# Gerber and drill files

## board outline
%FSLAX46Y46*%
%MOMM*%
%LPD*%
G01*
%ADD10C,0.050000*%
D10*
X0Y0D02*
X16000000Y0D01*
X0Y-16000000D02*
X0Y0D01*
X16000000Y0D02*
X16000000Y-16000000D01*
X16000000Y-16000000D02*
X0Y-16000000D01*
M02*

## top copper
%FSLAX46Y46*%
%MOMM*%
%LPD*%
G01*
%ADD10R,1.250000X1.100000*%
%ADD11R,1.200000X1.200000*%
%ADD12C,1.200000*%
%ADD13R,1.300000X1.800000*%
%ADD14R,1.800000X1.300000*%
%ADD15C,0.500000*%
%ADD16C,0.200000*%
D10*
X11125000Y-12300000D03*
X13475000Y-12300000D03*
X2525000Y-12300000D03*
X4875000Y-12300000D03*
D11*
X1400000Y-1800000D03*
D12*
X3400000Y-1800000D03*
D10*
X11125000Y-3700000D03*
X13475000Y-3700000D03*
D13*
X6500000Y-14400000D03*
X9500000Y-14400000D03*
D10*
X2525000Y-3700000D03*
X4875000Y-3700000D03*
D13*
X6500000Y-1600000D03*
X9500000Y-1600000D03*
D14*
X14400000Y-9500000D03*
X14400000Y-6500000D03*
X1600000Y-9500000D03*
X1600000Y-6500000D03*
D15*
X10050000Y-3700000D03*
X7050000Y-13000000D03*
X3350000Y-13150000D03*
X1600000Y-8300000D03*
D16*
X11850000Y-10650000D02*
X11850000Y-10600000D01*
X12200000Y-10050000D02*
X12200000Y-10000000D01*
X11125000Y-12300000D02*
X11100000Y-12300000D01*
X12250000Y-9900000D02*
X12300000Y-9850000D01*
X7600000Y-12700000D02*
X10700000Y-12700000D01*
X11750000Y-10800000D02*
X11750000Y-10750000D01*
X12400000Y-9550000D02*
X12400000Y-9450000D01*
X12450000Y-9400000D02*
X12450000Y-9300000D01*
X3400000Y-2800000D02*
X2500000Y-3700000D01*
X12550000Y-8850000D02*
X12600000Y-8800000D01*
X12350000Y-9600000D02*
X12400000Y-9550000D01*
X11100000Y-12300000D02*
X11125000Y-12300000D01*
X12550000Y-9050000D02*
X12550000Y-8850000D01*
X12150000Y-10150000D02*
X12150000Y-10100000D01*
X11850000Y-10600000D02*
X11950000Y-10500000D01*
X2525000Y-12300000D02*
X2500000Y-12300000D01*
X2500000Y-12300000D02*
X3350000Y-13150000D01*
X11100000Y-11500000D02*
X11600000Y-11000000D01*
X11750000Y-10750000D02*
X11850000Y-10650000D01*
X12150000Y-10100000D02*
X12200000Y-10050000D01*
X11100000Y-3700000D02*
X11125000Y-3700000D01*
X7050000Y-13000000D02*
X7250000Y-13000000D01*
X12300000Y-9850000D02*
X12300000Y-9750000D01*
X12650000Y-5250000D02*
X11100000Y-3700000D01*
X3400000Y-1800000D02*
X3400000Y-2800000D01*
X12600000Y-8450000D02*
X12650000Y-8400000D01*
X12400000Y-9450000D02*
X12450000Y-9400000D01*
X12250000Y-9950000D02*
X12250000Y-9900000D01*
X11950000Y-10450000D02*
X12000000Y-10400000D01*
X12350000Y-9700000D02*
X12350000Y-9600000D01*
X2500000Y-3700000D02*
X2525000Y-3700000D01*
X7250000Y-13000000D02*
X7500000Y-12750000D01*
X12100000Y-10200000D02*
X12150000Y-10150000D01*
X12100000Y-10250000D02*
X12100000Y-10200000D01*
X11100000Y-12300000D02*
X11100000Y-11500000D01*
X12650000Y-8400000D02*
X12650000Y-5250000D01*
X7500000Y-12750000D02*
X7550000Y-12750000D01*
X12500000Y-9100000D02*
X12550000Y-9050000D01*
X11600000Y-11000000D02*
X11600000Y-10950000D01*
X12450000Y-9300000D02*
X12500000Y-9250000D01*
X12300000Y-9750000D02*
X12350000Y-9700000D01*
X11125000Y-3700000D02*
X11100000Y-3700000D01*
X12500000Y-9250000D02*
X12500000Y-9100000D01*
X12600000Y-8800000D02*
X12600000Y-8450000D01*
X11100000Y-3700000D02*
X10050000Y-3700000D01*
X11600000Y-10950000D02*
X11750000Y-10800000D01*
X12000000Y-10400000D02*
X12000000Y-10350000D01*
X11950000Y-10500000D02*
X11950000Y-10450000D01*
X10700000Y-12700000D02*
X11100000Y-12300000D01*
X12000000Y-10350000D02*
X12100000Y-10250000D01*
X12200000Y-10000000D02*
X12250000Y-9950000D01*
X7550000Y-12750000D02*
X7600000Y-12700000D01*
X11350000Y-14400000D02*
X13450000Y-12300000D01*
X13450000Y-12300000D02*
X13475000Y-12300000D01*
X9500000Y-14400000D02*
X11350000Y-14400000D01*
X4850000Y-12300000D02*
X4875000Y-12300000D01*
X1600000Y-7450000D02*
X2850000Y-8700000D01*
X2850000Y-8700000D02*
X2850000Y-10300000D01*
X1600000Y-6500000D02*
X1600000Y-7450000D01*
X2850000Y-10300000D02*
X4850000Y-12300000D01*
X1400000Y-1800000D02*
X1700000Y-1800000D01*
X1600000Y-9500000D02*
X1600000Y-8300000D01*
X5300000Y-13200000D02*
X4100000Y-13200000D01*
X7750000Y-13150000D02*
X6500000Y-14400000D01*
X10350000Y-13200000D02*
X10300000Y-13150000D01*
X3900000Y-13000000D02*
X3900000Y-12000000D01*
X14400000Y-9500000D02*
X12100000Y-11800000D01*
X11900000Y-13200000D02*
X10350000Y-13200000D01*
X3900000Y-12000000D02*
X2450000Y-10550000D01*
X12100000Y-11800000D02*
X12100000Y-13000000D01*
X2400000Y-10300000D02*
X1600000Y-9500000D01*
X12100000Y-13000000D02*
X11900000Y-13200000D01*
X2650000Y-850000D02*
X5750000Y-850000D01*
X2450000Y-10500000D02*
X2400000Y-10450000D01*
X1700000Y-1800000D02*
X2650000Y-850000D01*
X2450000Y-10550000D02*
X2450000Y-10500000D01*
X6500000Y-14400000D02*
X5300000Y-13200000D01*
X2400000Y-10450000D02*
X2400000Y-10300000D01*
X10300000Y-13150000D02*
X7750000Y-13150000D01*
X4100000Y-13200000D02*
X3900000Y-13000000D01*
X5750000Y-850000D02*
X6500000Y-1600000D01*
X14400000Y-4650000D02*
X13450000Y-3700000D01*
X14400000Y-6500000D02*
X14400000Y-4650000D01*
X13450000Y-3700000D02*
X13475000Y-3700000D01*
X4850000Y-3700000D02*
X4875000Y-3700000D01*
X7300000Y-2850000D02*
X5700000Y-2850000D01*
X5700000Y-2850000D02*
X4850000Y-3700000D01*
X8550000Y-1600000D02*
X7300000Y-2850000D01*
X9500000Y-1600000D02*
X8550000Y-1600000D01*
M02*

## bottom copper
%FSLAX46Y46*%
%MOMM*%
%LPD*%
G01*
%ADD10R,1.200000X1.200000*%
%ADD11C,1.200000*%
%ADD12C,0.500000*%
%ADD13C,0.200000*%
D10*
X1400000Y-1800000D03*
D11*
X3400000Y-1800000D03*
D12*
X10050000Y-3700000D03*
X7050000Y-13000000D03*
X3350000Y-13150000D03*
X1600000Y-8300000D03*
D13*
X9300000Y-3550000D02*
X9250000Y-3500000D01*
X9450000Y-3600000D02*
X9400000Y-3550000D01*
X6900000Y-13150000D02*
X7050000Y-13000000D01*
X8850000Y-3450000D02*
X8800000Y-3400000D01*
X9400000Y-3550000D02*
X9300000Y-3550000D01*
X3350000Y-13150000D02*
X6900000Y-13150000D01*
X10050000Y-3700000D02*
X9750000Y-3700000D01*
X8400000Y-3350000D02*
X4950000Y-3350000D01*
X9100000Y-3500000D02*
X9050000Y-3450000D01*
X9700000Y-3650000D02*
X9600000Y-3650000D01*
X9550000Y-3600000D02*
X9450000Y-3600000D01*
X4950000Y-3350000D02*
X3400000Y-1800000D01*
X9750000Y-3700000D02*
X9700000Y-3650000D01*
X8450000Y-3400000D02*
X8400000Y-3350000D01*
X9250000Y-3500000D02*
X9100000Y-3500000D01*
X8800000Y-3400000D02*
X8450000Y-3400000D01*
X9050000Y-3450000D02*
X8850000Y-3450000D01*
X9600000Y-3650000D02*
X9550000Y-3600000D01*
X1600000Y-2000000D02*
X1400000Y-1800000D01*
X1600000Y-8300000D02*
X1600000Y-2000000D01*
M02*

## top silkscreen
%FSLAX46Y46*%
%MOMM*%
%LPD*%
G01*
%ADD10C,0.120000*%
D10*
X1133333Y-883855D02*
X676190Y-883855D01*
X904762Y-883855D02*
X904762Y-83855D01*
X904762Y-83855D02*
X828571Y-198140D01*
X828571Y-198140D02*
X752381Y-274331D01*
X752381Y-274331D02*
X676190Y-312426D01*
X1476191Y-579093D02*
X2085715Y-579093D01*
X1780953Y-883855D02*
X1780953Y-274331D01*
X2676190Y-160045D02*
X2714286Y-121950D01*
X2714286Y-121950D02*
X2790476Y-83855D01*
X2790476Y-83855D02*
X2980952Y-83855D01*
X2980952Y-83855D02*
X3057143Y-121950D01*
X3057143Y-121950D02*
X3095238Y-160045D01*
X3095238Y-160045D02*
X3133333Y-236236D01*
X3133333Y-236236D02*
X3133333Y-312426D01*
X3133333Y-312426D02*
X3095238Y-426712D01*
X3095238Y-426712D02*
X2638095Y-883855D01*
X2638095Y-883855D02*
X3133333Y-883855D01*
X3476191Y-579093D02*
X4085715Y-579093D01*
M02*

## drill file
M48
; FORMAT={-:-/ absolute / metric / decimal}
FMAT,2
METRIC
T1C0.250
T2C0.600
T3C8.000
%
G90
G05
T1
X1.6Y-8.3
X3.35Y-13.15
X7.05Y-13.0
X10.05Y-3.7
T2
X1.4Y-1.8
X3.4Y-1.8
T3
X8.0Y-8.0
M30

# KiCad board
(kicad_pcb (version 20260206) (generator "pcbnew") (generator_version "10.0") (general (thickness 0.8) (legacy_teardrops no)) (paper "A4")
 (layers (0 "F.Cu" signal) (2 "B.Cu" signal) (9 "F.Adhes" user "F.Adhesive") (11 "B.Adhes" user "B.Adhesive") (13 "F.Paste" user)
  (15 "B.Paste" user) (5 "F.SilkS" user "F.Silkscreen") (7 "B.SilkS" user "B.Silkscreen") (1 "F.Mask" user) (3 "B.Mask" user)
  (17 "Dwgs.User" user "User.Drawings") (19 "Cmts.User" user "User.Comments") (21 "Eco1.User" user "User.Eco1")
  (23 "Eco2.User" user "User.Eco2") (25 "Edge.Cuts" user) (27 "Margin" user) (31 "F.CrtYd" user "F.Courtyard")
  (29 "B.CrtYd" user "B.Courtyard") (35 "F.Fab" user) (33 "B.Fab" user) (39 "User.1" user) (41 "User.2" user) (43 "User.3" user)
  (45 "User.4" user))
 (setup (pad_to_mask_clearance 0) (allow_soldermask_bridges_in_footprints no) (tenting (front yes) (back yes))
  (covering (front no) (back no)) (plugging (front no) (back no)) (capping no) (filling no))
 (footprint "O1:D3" (layer "F.Cu") (at 12.3 12.3)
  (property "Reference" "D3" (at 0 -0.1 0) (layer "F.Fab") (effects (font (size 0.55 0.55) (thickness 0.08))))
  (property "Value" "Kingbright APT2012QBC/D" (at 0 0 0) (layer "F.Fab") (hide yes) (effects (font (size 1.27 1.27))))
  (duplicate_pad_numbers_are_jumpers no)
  (pad "1" smd rect (at -1.175 0) (size 1.25 1.1) (layers "F.Cu" "F.Mask" "F.Paste") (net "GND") (solder_mask_margin 0.025)
   (thermal_bridge_angle 45))
  (pad "2" smd rect (at 1.175 0) (size 1.25 1.1) (layers "F.Cu" "F.Mask" "F.Paste") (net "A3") (solder_mask_margin 0.025)
   (thermal_bridge_angle 45)))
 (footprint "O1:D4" (layer "F.Cu") (at 3.7 12.3)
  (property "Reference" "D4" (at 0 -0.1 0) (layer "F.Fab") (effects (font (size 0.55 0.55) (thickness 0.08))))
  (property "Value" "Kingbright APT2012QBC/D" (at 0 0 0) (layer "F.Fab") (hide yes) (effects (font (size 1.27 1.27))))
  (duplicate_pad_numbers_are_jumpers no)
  (pad "1" smd rect (at -1.175 0) (size 1.25 1.1) (layers "F.Cu" "F.Mask" "F.Paste") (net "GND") (solder_mask_margin 0.025)
   (thermal_bridge_angle 45))
  (pad "2" smd rect (at 1.175 0) (size 1.25 1.1) (layers "F.Cu" "F.Mask" "F.Paste") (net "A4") (solder_mask_margin 0.025)
   (thermal_bridge_angle 45)))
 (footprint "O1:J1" (layer "F.Cu") (at 2.4 1.8)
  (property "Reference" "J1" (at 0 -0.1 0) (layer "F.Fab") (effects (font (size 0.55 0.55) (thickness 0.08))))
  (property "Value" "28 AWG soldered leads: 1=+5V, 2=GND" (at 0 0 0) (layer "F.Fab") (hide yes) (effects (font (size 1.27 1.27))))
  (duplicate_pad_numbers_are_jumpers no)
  (pad "1" thru_hole rect (at -1 0) (size 1.2 1.2) (drill 0.6) (layers "*.Cu" "*.Mask") (remove_unused_layers no) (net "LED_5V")
   (solder_mask_margin 0.025) (thermal_bridge_angle 45))
  (pad "2" thru_hole circle (at 1 0) (size 1.2 1.2) (drill 0.6) (layers "*.Cu" "*.Mask") (remove_unused_layers no) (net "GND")
   (solder_mask_margin 0.025)))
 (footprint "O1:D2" (layer "F.Cu") (at 12.3 3.7)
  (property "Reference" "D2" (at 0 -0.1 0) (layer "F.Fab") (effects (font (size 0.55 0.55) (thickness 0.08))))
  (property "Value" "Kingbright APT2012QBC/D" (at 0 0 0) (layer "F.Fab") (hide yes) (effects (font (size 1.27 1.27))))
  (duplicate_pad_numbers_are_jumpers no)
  (pad "1" smd rect (at -1.175 0) (size 1.25 1.1) (layers "F.Cu" "F.Mask" "F.Paste") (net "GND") (solder_mask_margin 0.025)
   (thermal_bridge_angle 45))
  (pad "2" smd rect (at 1.175 0) (size 1.25 1.1) (layers "F.Cu" "F.Mask" "F.Paste") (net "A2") (solder_mask_margin 0.025)
   (thermal_bridge_angle 45)))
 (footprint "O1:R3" (layer "F.Cu") (at 8 14.4)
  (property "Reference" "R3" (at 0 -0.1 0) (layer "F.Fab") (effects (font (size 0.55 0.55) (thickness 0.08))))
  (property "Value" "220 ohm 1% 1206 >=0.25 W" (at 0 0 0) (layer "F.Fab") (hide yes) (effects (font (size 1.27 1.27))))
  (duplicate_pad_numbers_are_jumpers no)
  (pad "1" smd rect (at -1.5 0) (size 1.3 1.8) (layers "F.Cu" "F.Mask" "F.Paste") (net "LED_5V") (solder_mask_margin 0.025)
   (thermal_bridge_angle 45))
  (pad "2" smd rect (at 1.5 0) (size 1.3 1.8) (layers "F.Cu" "F.Mask" "F.Paste") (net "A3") (solder_mask_margin 0.025)
   (thermal_bridge_angle 45)))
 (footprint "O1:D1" (layer "F.Cu") (at 3.7 3.7)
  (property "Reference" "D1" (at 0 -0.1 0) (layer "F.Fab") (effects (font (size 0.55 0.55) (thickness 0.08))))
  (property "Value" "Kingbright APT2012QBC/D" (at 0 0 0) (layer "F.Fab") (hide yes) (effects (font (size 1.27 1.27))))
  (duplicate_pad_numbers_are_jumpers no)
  (pad "1" smd rect (at -1.175 0) (size 1.25 1.1) (layers "F.Cu" "F.Mask" "F.Paste") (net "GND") (solder_mask_margin 0.025)
   (thermal_bridge_angle 45))
  (pad "2" smd rect (at 1.175 0) (size 1.25 1.1) (layers "F.Cu" "F.Mask" "F.Paste") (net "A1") (solder_mask_margin 0.025)
   (thermal_bridge_angle 45)))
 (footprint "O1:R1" (layer "F.Cu") (at 8 1.6)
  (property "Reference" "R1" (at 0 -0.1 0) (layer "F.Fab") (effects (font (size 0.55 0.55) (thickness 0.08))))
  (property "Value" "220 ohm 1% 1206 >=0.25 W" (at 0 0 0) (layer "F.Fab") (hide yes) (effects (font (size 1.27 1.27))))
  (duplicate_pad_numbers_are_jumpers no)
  (pad "1" smd rect (at -1.5 0) (size 1.3 1.8) (layers "F.Cu" "F.Mask" "F.Paste") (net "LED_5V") (solder_mask_margin 0.025)
   (thermal_bridge_angle 45))
  (pad "2" smd rect (at 1.5 0) (size 1.3 1.8) (layers "F.Cu" "F.Mask" "F.Paste") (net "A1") (solder_mask_margin 0.025)
   (thermal_bridge_angle 45)))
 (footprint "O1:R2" (layer "F.Cu") (at 14.4 8 90)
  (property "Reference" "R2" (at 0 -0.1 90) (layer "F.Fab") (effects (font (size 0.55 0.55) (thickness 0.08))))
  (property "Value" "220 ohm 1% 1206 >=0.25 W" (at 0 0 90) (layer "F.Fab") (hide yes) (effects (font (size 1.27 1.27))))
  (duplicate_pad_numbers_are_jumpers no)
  (pad "1" smd rect (at -1.5 0 90) (size 1.3 1.8) (layers "F.Cu" "F.Mask" "F.Paste") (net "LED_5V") (solder_mask_margin 0.025)
   (thermal_bridge_angle 45))
  (pad "2" smd rect (at 1.5 0 90) (size 1.3 1.8) (layers "F.Cu" "F.Mask" "F.Paste") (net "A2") (solder_mask_margin 0.025)
   (thermal_bridge_angle 45)))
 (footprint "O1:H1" (layer "F.Cu") (at 8 8)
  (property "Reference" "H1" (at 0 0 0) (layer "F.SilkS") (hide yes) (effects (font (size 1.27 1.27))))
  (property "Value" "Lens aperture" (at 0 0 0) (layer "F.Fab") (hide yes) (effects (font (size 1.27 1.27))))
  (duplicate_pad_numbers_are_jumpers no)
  (pad "" np_thru_hole circle (at 0 0) (size 8 8) (drill 8) (layers "*.Cu" "*.Mask")))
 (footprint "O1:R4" (layer "F.Cu") (at 1.6 8 90)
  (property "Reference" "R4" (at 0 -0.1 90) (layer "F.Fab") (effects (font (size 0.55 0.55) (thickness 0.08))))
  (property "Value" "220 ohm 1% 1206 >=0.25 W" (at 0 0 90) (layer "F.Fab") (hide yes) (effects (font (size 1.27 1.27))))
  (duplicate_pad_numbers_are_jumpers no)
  (pad "1" smd rect (at -1.5 0 90) (size 1.3 1.8) (layers "F.Cu" "F.Mask" "F.Paste") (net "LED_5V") (solder_mask_margin 0.025)
   (thermal_bridge_angle 45))
  (pad "2" smd rect (at 1.5 0 90) (size 1.3 1.8) (layers "F.Cu" "F.Mask" "F.Paste") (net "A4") (solder_mask_margin 0.025)
   (thermal_bridge_angle 45)))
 (gr_line (start 0 0) (end 16 0) (stroke (width 0.05) (type default)) (layer "Edge.Cuts"))
 (gr_line (start 0 16) (end 0 0) (stroke (width 0.05) (type default)) (layer "Edge.Cuts"))
 (gr_line (start 16 0) (end 16 16) (stroke (width 0.05) (type default)) (layer "Edge.Cuts"))
 (gr_line (start 16 16) (end 0 16) (stroke (width 0.05) (type default)) (layer "Edge.Cuts"))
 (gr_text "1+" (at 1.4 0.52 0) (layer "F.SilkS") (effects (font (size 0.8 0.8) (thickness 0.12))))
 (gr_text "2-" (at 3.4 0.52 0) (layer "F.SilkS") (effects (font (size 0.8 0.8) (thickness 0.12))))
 (segment (start 4.85 3.7) (end 4.875 3.7) (width 0.2) (layer "F.Cu") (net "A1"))
 (segment (start 7.3 2.85) (end 5.7 2.85) (width 0.2) (layer "F.Cu") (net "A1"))
 (segment (start 5.7 2.85) (end 4.85 3.7) (width 0.2) (layer "F.Cu") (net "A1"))
 (segment (start 8.55 1.6) (end 7.3 2.85) (width 0.2) (layer "F.Cu") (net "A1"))
 (segment (start 9.5 1.6) (end 8.55 1.6) (width 0.2) (layer "F.Cu") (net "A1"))
 (segment (start 14.4 4.65) (end 13.45 3.7) (width 0.2) (layer "F.Cu") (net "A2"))
 (segment (start 14.4 6.5) (end 14.4 4.65) (width 0.2) (layer "F.Cu") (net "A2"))
 (segment (start 13.45 3.7) (end 13.475 3.7) (width 0.2) (layer "F.Cu") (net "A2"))
 (segment (start 11.35 14.4) (end 13.45 12.3) (width 0.2) (layer "F.Cu") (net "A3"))
 (segment (start 13.45 12.3) (end 13.475 12.3) (width 0.2) (layer "F.Cu") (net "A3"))
 (segment (start 9.5 14.4) (end 11.35 14.4) (width 0.2) (layer "F.Cu") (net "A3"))
 (segment (start 4.85 12.3) (end 4.875 12.3) (width 0.2) (layer "F.Cu") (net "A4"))
 (segment (start 1.6 7.45) (end 2.85 8.7) (width 0.2) (layer "F.Cu") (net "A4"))
 (segment (start 2.85 8.7) (end 2.85 10.3) (width 0.2) (layer "F.Cu") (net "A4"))
 (segment (start 1.6 6.5) (end 1.6 7.45) (width 0.2) (layer "F.Cu") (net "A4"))
 (segment (start 2.85 10.3) (end 4.85 12.3) (width 0.2) (layer "F.Cu") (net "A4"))
 (segment (start 11.85 10.65) (end 11.85 10.6) (width 0.2) (layer "F.Cu") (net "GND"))
 (segment (start 12.2 10.05) (end 12.2 10) (width 0.2) (layer "F.Cu") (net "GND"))
 (segment (start 11.125 12.3) (end 11.1 12.3) (width 0.2) (layer "F.Cu") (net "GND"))
 (segment (start 12.25 9.9) (end 12.3 9.85) (width 0.2) (layer "F.Cu") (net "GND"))
 (segment (start 7.6 12.7) (end 10.7 12.7) (width 0.2) (layer "F.Cu") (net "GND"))
 (segment (start 11.75 10.8) (end 11.75 10.75) (width 0.2) (layer "F.Cu") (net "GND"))
 (segment (start 12.4 9.55) (end 12.4 9.45) (width 0.2) (layer "F.Cu") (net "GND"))
 (segment (start 12.45 9.4) (end 12.45 9.3) (width 0.2) (layer "F.Cu") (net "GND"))
 (segment (start 3.4 2.8) (end 2.5 3.7) (width 0.2) (layer "F.Cu") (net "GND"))
 (segment (start 12.55 8.85) (end 12.6 8.8) (width 0.2) (layer "F.Cu") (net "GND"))
 (segment (start 12.35 9.6) (end 12.4 9.55) (width 0.2) (layer "F.Cu") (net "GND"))
 (segment (start 11.1 12.3) (end 11.125 12.3) (width 0.2) (layer "F.Cu") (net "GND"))
 (segment (start 12.55 9.05) (end 12.55 8.85) (width 0.2) (layer "F.Cu") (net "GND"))
 (segment (start 12.15 10.15) (end 12.15 10.1) (width 0.2) (layer "F.Cu") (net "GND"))
 (segment (start 11.85 10.6) (end 11.95 10.5) (width 0.2) (layer "F.Cu") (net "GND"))
 (segment (start 2.525 12.3) (end 2.5 12.3) (width 0.2) (layer "F.Cu") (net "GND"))
 (segment (start 2.5 12.3) (end 3.35 13.15) (width 0.2) (layer "F.Cu") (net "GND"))
 (segment (start 11.1 11.5) (end 11.6 11) (width 0.2) (layer "F.Cu") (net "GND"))
 (segment (start 11.75 10.75) (end 11.85 10.65) (width 0.2) (layer "F.Cu") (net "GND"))
 (segment (start 12.15 10.1) (end 12.2 10.05) (width 0.2) (layer "F.Cu") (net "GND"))
 (segment (start 11.1 3.7) (end 11.125 3.7) (width 0.2) (layer "F.Cu") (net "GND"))
 (segment (start 7.05 13) (end 7.25 13) (width 0.2) (layer "F.Cu") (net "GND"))
 (segment (start 12.3 9.85) (end 12.3 9.75) (width 0.2) (layer "F.Cu") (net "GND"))
 (segment (start 12.65 5.25) (end 11.1 3.7) (width 0.2) (layer "F.Cu") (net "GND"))
 (segment (start 3.4 1.8) (end 3.4 2.8) (width 0.2) (layer "F.Cu") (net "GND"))
 (segment (start 12.6 8.45) (end 12.65 8.4) (width 0.2) (layer "F.Cu") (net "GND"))
 (segment (start 12.4 9.45) (end 12.45 9.4) (width 0.2) (layer "F.Cu") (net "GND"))
 (segment (start 12.25 9.95) (end 12.25 9.9) (width 0.2) (layer "F.Cu") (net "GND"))
 (segment (start 11.95 10.45) (end 12 10.4) (width 0.2) (layer "F.Cu") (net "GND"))
 (segment (start 12.35 9.7) (end 12.35 9.6) (width 0.2) (layer "F.Cu") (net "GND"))
 (segment (start 2.5 3.7) (end 2.525 3.7) (width 0.2) (layer "F.Cu") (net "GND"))
 (segment (start 7.25 13) (end 7.5 12.75) (width 0.2) (layer "F.Cu") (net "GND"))
 (segment (start 12.1 10.2) (end 12.15 10.15) (width 0.2) (layer "F.Cu") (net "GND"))
 (segment (start 12.1 10.25) (end 12.1 10.2) (width 0.2) (layer "F.Cu") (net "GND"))
 (segment (start 11.1 12.3) (end 11.1 11.5) (width 0.2) (layer "F.Cu") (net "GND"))
 (segment (start 12.65 8.4) (end 12.65 5.25) (width 0.2) (layer "F.Cu") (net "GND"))
 (segment (start 7.5 12.75) (end 7.55 12.75) (width 0.2) (layer "F.Cu") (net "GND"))
 (segment (start 12.5 9.1) (end 12.55 9.05) (width 0.2) (layer "F.Cu") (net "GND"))
 (segment (start 11.6 11) (end 11.6 10.95) (width 0.2) (layer "F.Cu") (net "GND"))
 (segment (start 12.45 9.3) (end 12.5 9.25) (width 0.2) (layer "F.Cu") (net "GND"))
 (segment (start 12.3 9.75) (end 12.35 9.7) (width 0.2) (layer "F.Cu") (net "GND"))
 (segment (start 11.125 3.7) (end 11.1 3.7) (width 0.2) (layer "F.Cu") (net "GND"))
 (segment (start 12.5 9.25) (end 12.5 9.1) (width 0.2) (layer "F.Cu") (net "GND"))
 (segment (start 12.6 8.8) (end 12.6 8.45) (width 0.2) (layer "F.Cu") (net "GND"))
 (segment (start 11.1 3.7) (end 10.05 3.7) (width 0.2) (layer "F.Cu") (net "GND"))
 (segment (start 11.6 10.95) (end 11.75 10.8) (width 0.2) (layer "F.Cu") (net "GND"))
 (segment (start 12 10.4) (end 12 10.35) (width 0.2) (layer "F.Cu") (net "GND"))
 (segment (start 11.95 10.5) (end 11.95 10.45) (width 0.2) (layer "F.Cu") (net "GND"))
 (segment (start 10.7 12.7) (end 11.1 12.3) (width 0.2) (layer "F.Cu") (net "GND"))
 (segment (start 12 10.35) (end 12.1 10.25) (width 0.2) (layer "F.Cu") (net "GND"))
 (segment (start 12.2 10) (end 12.25 9.95) (width 0.2) (layer "F.Cu") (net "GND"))
 (segment (start 7.55 12.75) (end 7.6 12.7) (width 0.2) (layer "F.Cu") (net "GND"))
 (via (at 10.05 3.7) (size 0.5) (drill 0.25) (layers "F.Cu" "B.Cu") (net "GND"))
 (via (at 7.05 13) (size 0.5) (drill 0.25) (layers "F.Cu" "B.Cu") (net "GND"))
 (via (at 3.35 13.15) (size 0.5) (drill 0.25) (layers "F.Cu" "B.Cu") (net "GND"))
 (segment (start 9.3 3.55) (end 9.25 3.5) (width 0.2) (layer "B.Cu") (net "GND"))
 (segment (start 9.45 3.6) (end 9.4 3.55) (width 0.2) (layer "B.Cu") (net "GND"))
 (segment (start 6.9 13.15) (end 7.05 13) (width 0.2) (layer "B.Cu") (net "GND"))
 (segment (start 8.85 3.45) (end 8.8 3.4) (width 0.2) (layer "B.Cu") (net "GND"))
 (segment (start 9.4 3.55) (end 9.3 3.55) (width 0.2) (layer "B.Cu") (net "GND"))
 (segment (start 3.35 13.15) (end 6.9 13.15) (width 0.2) (layer "B.Cu") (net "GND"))
 (segment (start 10.05 3.7) (end 9.75 3.7) (width 0.2) (layer "B.Cu") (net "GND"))
 (segment (start 8.4 3.35) (end 4.95 3.35) (width 0.2) (layer "B.Cu") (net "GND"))
 (segment (start 9.1 3.5) (end 9.05 3.45) (width 0.2) (layer "B.Cu") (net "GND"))
 (segment (start 9.7 3.65) (end 9.6 3.65) (width 0.2) (layer "B.Cu") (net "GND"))
 (segment (start 9.55 3.6) (end 9.45 3.6) (width 0.2) (layer "B.Cu") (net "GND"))
 (segment (start 4.95 3.35) (end 3.4 1.8) (width 0.2) (layer "B.Cu") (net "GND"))
 (segment (start 9.75 3.7) (end 9.7 3.65) (width 0.2) (layer "B.Cu") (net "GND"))
 (segment (start 8.45 3.4) (end 8.4 3.35) (width 0.2) (layer "B.Cu") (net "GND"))
 (segment (start 9.25 3.5) (end 9.1 3.5) (width 0.2) (layer "B.Cu") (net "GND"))
 (segment (start 8.8 3.4) (end 8.45 3.4) (width 0.2) (layer "B.Cu") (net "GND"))
 (segment (start 9.05 3.45) (end 8.85 3.45) (width 0.2) (layer "B.Cu") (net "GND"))
 (segment (start 9.6 3.65) (end 9.55 3.6) (width 0.2) (layer "B.Cu") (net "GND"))
 (segment (start 1.4 1.8) (end 1.7 1.8) (width 0.2) (layer "F.Cu") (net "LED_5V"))
 (segment (start 1.6 9.5) (end 1.6 8.3) (width 0.2) (layer "F.Cu") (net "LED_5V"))
 (segment (start 5.3 13.2) (end 4.1 13.2) (width 0.2) (layer "F.Cu") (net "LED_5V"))
 (segment (start 7.75 13.15) (end 6.5 14.4) (width 0.2) (layer "F.Cu") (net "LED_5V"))
 (segment (start 10.35 13.2) (end 10.3 13.15) (width 0.2) (layer "F.Cu") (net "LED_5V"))
 (segment (start 3.9 13) (end 3.9 12) (width 0.2) (layer "F.Cu") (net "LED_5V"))
 (segment (start 14.4 9.5) (end 12.1 11.8) (width 0.2) (layer "F.Cu") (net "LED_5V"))
 (segment (start 11.9 13.2) (end 10.35 13.2) (width 0.2) (layer "F.Cu") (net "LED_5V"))
 (segment (start 3.9 12) (end 2.45 10.55) (width 0.2) (layer "F.Cu") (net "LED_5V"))
 (segment (start 12.1 11.8) (end 12.1 13) (width 0.2) (layer "F.Cu") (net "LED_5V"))
 (segment (start 2.4 10.3) (end 1.6 9.5) (width 0.2) (layer "F.Cu") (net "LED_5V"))
 (segment (start 12.1 13) (end 11.9 13.2) (width 0.2) (layer "F.Cu") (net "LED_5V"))
 (segment (start 2.65 0.85) (end 5.75 0.85) (width 0.2) (layer "F.Cu") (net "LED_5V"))
 (segment (start 2.45 10.5) (end 2.4 10.45) (width 0.2) (layer "F.Cu") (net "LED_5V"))
 (segment (start 1.7 1.8) (end 2.65 0.85) (width 0.2) (layer "F.Cu") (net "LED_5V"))
 (segment (start 2.45 10.55) (end 2.45 10.5) (width 0.2) (layer "F.Cu") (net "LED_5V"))
 (segment (start 6.5 14.4) (end 5.3 13.2) (width 0.2) (layer "F.Cu") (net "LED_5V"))
 (segment (start 2.4 10.45) (end 2.4 10.3) (width 0.2) (layer "F.Cu") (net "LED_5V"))
 (segment (start 10.3 13.15) (end 7.75 13.15) (width 0.2) (layer "F.Cu") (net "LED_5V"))
 (segment (start 4.1 13.2) (end 3.9 13) (width 0.2) (layer "F.Cu") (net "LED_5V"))
 (segment (start 5.75 0.85) (end 6.5 1.6) (width 0.2) (layer "F.Cu") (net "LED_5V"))
 (via (at 1.6 8.3) (size 0.5) (drill 0.25) (layers "F.Cu" "B.Cu") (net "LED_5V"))
 (segment (start 1.6 2) (end 1.4 1.8) (width 0.2) (layer "B.Cu") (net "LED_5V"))
 (segment (start 1.6 8.3) (end 1.6 2) (width 0.2) (layer "B.Cu") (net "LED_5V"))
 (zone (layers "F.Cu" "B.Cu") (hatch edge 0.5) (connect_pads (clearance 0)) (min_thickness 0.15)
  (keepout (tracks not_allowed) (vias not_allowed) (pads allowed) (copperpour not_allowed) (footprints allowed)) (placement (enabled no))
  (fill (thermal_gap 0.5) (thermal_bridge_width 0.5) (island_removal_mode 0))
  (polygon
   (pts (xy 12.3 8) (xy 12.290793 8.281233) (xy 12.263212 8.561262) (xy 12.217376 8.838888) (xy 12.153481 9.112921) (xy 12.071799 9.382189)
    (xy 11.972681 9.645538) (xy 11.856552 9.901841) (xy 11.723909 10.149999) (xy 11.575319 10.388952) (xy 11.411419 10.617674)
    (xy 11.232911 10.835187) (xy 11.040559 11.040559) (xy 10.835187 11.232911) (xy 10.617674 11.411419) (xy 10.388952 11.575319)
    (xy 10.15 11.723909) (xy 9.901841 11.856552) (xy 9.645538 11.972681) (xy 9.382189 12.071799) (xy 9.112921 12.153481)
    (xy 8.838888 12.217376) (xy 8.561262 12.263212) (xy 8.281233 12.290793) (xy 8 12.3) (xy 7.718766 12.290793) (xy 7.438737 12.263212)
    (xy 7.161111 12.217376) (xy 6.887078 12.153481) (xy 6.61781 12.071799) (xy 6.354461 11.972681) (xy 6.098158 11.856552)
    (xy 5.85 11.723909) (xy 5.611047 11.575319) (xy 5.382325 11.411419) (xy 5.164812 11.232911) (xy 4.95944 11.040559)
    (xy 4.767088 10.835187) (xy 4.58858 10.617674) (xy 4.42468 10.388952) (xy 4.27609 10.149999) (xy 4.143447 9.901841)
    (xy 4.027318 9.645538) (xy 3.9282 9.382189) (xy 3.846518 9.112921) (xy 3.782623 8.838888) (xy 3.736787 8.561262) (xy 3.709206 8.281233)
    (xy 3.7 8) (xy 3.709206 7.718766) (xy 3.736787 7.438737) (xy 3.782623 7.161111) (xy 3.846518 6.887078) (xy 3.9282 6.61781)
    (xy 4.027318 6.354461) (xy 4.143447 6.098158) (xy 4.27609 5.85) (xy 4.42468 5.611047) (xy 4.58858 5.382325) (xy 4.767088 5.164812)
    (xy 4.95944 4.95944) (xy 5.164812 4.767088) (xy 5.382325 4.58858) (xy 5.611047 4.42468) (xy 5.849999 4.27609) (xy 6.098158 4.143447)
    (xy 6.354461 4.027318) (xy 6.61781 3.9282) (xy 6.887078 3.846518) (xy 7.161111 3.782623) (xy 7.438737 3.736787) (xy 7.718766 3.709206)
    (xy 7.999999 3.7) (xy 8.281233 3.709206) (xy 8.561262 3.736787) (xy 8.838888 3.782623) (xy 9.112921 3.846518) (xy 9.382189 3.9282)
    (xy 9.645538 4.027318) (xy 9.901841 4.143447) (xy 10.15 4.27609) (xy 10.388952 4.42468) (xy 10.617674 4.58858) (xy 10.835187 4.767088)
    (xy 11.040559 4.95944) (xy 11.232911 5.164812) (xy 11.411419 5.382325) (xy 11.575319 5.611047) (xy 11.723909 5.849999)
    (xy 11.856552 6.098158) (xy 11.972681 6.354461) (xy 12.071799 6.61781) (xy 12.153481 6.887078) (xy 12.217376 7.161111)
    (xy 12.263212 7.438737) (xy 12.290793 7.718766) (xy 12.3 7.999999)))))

